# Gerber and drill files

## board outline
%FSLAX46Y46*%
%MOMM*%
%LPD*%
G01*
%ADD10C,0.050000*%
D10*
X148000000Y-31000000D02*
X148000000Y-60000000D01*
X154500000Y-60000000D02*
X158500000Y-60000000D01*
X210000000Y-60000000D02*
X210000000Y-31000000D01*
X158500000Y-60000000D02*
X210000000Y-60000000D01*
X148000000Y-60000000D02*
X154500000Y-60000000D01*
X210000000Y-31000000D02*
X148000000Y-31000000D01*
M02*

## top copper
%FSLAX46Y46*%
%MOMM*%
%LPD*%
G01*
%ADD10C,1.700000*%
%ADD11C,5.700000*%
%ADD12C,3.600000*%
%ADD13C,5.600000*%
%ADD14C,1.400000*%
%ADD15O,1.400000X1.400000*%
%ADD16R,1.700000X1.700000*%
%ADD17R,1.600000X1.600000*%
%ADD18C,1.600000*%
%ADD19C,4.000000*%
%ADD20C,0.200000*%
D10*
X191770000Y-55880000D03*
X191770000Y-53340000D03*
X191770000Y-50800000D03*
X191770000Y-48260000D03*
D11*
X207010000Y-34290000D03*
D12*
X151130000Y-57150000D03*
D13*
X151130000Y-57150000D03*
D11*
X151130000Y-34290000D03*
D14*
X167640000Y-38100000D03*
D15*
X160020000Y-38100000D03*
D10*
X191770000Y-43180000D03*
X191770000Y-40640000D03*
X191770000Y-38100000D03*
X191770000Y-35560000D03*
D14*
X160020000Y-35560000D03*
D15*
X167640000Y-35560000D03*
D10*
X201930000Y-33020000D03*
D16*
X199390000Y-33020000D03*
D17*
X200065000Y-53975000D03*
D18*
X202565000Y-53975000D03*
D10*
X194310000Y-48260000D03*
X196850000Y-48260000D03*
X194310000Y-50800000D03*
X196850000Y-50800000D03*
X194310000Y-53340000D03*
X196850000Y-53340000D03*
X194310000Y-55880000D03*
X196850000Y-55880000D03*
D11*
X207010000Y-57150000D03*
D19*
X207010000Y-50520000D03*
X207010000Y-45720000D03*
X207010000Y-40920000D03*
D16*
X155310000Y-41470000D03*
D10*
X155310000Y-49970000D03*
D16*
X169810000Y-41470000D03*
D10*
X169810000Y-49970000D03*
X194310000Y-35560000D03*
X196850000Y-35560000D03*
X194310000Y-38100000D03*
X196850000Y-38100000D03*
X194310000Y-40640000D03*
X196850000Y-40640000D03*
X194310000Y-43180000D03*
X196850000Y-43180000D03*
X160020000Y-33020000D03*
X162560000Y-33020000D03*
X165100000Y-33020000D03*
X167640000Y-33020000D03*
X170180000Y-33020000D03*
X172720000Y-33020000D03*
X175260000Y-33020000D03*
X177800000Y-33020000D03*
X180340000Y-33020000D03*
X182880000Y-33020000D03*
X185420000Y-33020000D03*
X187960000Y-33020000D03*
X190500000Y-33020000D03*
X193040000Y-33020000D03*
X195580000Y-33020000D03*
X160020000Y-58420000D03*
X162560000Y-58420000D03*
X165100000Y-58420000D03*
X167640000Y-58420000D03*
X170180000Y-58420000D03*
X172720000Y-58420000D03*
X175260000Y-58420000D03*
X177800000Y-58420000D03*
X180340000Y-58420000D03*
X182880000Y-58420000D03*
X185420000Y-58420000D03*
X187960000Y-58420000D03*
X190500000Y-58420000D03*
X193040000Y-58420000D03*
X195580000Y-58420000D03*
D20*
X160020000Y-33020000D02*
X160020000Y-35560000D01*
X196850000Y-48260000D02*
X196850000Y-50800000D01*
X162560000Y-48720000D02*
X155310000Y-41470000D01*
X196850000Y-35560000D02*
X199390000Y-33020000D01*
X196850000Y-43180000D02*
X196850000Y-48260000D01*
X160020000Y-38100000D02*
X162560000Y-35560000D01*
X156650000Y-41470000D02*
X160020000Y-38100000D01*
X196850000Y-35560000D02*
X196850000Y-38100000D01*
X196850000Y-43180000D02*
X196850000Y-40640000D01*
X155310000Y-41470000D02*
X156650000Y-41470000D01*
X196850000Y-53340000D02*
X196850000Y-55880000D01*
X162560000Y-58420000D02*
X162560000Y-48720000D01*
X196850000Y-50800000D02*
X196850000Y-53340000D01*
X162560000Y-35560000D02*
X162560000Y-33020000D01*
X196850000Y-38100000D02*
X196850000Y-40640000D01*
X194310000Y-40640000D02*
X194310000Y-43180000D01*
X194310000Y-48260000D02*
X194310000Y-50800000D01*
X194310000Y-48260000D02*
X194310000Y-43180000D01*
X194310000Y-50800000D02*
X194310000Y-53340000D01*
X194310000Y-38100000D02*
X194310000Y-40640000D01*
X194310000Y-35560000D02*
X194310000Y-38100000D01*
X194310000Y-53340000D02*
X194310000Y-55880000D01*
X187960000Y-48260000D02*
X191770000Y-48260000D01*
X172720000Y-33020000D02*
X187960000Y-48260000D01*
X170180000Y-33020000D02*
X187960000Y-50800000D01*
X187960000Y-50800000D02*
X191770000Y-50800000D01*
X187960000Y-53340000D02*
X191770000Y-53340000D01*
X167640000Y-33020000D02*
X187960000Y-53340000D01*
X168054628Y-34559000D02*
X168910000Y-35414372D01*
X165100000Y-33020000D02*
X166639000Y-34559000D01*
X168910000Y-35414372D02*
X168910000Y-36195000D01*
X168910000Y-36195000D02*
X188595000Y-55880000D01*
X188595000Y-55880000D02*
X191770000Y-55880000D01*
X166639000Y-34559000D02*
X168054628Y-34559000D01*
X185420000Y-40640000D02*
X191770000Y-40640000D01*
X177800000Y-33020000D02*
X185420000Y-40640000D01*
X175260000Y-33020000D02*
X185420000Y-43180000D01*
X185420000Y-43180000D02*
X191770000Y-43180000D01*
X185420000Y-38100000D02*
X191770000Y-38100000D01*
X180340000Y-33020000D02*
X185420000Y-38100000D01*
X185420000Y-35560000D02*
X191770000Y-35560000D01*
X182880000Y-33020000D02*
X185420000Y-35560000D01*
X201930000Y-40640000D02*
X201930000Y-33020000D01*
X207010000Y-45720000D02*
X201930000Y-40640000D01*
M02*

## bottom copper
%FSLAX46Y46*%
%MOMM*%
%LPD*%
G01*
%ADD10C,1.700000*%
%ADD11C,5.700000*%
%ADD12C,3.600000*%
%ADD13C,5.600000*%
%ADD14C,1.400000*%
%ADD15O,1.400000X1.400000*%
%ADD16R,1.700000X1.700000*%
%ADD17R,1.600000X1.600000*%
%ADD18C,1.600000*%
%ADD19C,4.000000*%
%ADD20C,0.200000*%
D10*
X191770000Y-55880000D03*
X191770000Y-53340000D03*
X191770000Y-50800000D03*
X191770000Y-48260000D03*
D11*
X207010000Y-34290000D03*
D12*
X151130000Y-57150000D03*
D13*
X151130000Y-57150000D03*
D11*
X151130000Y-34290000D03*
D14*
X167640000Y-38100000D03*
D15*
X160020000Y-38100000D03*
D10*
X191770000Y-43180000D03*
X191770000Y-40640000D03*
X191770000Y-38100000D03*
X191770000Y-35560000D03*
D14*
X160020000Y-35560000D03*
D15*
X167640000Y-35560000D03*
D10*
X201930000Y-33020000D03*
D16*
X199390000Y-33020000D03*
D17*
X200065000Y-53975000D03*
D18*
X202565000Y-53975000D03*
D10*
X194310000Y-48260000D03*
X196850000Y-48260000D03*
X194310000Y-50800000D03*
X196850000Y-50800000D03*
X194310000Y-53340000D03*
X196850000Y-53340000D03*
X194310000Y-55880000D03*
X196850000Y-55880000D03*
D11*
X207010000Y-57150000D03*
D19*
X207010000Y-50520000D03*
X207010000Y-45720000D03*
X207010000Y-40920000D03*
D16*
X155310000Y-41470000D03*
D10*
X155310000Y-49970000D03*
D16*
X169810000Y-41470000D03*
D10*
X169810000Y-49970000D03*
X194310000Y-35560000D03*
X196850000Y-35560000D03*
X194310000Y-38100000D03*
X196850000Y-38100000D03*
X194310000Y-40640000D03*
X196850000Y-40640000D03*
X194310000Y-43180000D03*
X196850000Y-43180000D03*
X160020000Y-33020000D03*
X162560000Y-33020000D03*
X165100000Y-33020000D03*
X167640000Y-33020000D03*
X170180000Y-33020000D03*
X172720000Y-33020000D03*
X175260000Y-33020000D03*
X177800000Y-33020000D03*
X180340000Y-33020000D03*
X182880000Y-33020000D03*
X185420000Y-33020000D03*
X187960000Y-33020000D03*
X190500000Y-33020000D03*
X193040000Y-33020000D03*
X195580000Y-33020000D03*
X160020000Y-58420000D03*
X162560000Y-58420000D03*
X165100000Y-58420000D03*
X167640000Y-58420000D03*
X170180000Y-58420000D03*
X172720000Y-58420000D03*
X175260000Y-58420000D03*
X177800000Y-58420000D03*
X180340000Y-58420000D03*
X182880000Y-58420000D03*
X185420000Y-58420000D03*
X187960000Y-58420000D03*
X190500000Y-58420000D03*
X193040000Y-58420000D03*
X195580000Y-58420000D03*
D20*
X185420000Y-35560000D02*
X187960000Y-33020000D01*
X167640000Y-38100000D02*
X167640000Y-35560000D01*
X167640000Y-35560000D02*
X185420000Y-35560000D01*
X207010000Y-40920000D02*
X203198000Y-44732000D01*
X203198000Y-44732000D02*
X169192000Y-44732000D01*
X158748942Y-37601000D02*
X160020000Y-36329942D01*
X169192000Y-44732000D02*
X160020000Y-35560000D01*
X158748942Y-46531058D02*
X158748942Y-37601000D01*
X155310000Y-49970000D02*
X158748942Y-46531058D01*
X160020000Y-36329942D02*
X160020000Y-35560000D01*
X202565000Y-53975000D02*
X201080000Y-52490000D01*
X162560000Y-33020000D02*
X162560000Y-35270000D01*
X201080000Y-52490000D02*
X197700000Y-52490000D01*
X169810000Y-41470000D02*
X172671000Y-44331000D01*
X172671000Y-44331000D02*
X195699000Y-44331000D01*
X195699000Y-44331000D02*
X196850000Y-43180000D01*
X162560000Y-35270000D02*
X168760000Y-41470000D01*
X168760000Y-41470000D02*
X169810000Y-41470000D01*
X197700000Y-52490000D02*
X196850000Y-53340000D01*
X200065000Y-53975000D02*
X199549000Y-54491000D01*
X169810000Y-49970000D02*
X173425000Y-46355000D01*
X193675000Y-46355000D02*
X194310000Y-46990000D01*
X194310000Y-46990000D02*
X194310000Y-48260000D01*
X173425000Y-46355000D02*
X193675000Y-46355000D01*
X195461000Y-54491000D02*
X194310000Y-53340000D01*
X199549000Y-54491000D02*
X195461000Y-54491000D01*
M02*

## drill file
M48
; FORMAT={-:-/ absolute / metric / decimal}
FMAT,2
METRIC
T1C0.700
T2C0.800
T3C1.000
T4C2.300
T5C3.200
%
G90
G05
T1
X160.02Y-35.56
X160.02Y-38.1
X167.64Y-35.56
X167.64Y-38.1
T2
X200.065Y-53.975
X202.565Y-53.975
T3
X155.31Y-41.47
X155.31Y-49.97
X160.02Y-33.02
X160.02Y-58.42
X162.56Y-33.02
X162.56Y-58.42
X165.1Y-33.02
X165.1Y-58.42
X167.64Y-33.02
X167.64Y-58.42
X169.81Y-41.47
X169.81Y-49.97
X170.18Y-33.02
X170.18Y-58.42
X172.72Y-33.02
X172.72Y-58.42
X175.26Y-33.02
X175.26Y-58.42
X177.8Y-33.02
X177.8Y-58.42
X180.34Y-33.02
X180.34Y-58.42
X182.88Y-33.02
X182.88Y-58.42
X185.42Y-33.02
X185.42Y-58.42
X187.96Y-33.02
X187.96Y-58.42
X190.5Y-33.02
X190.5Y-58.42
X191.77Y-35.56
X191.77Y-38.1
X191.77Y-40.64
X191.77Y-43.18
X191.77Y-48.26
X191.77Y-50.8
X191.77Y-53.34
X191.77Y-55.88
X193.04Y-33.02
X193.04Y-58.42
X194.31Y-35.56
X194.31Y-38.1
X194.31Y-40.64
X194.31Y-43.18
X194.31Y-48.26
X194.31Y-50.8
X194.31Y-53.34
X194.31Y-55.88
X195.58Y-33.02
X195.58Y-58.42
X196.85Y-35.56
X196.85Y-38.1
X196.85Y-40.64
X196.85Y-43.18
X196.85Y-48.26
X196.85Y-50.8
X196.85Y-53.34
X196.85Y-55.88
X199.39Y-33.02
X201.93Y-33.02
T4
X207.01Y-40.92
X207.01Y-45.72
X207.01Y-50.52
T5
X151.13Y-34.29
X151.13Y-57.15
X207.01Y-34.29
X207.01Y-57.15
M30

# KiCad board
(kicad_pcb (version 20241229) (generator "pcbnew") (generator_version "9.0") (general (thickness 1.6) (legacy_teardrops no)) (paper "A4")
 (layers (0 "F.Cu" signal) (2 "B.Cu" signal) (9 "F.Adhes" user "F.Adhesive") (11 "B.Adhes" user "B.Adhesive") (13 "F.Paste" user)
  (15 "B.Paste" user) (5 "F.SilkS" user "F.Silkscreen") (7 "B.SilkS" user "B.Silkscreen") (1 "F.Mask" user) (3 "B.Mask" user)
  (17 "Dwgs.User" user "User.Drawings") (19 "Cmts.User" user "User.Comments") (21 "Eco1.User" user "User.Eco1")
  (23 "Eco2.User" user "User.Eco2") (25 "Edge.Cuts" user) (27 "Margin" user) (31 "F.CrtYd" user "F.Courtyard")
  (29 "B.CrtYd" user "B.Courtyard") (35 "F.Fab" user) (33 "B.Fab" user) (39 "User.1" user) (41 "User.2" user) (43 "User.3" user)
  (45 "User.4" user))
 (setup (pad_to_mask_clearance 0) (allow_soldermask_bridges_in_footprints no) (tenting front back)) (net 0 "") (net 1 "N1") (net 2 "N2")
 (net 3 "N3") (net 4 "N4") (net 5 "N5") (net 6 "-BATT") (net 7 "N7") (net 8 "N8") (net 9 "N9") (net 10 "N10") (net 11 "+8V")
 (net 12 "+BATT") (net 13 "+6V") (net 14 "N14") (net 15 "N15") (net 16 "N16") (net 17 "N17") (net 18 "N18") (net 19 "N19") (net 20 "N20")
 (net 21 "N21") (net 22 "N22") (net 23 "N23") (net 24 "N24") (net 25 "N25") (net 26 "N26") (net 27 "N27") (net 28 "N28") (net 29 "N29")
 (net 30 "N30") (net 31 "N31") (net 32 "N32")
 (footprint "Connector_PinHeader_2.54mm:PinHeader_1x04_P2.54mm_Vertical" (layer "F.Cu") (at 191.77 55.88 180)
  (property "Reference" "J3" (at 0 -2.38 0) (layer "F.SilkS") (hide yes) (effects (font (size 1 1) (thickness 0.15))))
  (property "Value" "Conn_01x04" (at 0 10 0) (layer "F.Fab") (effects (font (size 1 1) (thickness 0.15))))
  (pad "1" thru_hole circle (at 0 0 180) (size 1.7 1.7) (drill 1) (layers "*.Cu" "*.Mask") (remove_unused_layers no) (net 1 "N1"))
  (pad "2" thru_hole circle (at 0 2.54 180) (size 1.7 1.7) (drill 1) (layers "*.Cu" "*.Mask") (remove_unused_layers no) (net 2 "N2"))
  (pad "3" thru_hole circle (at 0 5.08 180) (size 1.7 1.7) (drill 1) (layers "*.Cu" "*.Mask") (remove_unused_layers no) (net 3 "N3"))
  (pad "4" thru_hole circle (at 0 7.62 180) (size 1.7 1.7) (drill 1) (layers "*.Cu" "*.Mask") (remove_unused_layers no) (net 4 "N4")))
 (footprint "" (layer "F.Cu") (at 207.01 34.29)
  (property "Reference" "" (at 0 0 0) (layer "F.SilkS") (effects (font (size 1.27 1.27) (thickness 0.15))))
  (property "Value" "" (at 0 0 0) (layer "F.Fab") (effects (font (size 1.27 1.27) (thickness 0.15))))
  (pad "1" thru_hole circle (at 0 0) (size 5.7 5.7) (drill 3.2) (layers "*.Cu" "*.Mask") (remove_unused_layers no)))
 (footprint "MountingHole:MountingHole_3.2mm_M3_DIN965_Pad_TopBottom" (layer "F.Cu") (at 151.13 57.15)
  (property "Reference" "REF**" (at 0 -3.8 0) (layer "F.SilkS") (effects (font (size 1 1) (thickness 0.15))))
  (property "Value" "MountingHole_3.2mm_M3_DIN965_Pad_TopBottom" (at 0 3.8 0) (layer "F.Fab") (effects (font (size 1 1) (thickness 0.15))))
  (pad "1" thru_hole circle (at 0 0) (size 3.6 3.6) (drill 3.2) (layers "*.Cu" "*.Mask") (remove_unused_layers no))
  (pad "1" connect circle (at 0 0) (size 5.6 5.6) (layers "F.Cu" "F.Mask"))
  (pad "1" connect circle (at 0 0) (size 5.6 5.6) (layers "B.Cu" "B.Mask")))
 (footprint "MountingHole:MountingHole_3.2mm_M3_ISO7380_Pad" (layer "F.Cu") (at 151.13 34.29)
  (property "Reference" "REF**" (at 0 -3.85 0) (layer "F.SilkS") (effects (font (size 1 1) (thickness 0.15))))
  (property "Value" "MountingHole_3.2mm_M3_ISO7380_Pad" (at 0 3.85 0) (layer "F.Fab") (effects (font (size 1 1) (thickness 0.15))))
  (pad "1" thru_hole circle (at 0 0) (size 5.7 5.7) (drill 3.2) (layers "*.Cu" "*.Mask") (remove_unused_layers no)))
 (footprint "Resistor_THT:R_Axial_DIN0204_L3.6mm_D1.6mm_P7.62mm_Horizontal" (layer "F.Cu") (at 167.64 38.1 180)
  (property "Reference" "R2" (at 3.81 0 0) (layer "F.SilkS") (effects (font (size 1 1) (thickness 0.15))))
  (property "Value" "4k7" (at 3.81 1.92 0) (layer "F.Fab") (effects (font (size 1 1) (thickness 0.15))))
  (pad "1" thru_hole circle (at 0 0 180) (size 1.4 1.4) (drill 0.7) (layers "*.Cu" "*.Mask") (remove_unused_layers no) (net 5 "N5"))
  (pad "2" thru_hole oval (at 7.62 0 180) (size 1.4 1.4) (drill 0.7) (layers "*.Cu" "*.Mask") (remove_unused_layers no) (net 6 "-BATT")))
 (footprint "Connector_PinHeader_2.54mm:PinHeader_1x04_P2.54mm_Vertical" (layer "F.Cu") (at 191.77 43.18 180)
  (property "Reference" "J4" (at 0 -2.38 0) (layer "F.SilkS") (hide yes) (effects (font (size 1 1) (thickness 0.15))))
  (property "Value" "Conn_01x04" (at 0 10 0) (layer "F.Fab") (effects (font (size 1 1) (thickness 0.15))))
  (pad "1" thru_hole circle (at 0 0 180) (size 1.7 1.7) (drill 1) (layers "*.Cu" "*.Mask") (remove_unused_layers no) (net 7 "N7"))
  (pad "2" thru_hole circle (at 0 2.54 180) (size 1.7 1.7) (drill 1) (layers "*.Cu" "*.Mask") (remove_unused_layers no) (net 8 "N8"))
  (pad "3" thru_hole circle (at 0 5.08 180) (size 1.7 1.7) (drill 1) (layers "*.Cu" "*.Mask") (remove_unused_layers no) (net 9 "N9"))
  (pad "4" thru_hole circle (at 0 7.62 180) (size 1.7 1.7) (drill 1) (layers "*.Cu" "*.Mask") (remove_unused_layers no) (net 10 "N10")))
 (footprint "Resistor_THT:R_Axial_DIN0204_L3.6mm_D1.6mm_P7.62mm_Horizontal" (layer "F.Cu") (at 160.02 35.56)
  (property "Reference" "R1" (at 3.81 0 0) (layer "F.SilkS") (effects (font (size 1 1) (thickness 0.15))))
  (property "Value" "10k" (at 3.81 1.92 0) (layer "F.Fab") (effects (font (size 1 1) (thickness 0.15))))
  (pad "1" thru_hole circle (at 0 0) (size 1.4 1.4) (drill 0.7) (layers "*.Cu" "*.Mask") (remove_unused_layers no) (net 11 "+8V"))
  (pad "2" thru_hole oval (at 7.62 0) (size 1.4 1.4) (drill 0.7) (layers "*.Cu" "*.Mask") (remove_unused_layers no) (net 5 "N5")))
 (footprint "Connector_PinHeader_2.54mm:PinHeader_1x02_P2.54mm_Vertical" (layer "F.Cu") (at 201.93 33.02 -90)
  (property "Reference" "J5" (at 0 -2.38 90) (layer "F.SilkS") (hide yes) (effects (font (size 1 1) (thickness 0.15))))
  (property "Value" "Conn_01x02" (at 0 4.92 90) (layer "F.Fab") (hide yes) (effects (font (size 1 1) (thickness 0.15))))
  (pad "1" thru_hole circle (at 0 0 270) (size 1.7 1.7) (drill 1) (layers "*.Cu" "*.Mask") (remove_unused_layers no) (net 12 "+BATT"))
  (pad "2" thru_hole rect (at 0 2.54 270) (size 1.7 1.7) (drill 1) (layers "*.Cu" "*.Mask") (remove_unused_layers no) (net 6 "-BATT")))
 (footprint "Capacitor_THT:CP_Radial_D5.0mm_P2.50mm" (layer "F.Cu") (at 200.065 53.975)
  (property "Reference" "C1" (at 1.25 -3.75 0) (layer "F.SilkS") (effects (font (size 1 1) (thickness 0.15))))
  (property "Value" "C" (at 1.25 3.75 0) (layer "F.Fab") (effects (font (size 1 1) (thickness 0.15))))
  (pad "1" thru_hole rect (at 0 0) (size 1.6 1.6) (drill 0.8) (layers "*.Cu" "*.Mask") (remove_unused_layers no) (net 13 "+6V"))
  (pad "2" thru_hole circle (at 2.5 0) (size 1.6 1.6) (drill 0.8) (layers "*.Cu" "*.Mask") (remove_unused_layers no) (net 6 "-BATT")))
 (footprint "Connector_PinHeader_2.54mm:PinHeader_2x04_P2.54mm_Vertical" (layer "F.Cu") (at 194.31 48.26)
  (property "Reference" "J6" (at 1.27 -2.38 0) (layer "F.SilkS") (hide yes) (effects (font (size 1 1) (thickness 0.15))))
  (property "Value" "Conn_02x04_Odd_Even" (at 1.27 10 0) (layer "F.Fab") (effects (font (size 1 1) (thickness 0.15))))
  (pad "1" thru_hole circle (at 0 0) (size 1.7 1.7) (drill 1) (layers "*.Cu" "*.Mask") (remove_unused_layers no) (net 13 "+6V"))
  (pad "2" thru_hole circle (at 2.54 0) (size 1.7 1.7) (drill 1) (layers "*.Cu" "*.Mask") (remove_unused_layers no) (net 6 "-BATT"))
  (pad "3" thru_hole circle (at 0 2.54) (size 1.7 1.7) (drill 1) (layers "*.Cu" "*.Mask") (remove_unused_layers no) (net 13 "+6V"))
  (pad "4" thru_hole circle (at 2.54 2.54) (size 1.7 1.7) (drill 1) (layers "*.Cu" "*.Mask") (remove_unused_layers no) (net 6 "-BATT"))
  (pad "5" thru_hole circle (at 0 5.08) (size 1.7 1.7) (drill 1) (layers "*.Cu" "*.Mask") (remove_unused_layers no) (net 13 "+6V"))
  (pad "6" thru_hole circle (at 2.54 5.08) (size 1.7 1.7) (drill 1) (layers "*.Cu" "*.Mask") (remove_unused_layers no) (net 6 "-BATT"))
  (pad "7" thru_hole circle (at 0 7.62) (size 1.7 1.7) (drill 1) (layers "*.Cu" "*.Mask") (remove_unused_layers no) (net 13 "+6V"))
  (pad "8" thru_hole circle (at 2.54 7.62) (size 1.7 1.7) (drill 1) (layers "*.Cu" "*.Mask") (remove_unused_layers no) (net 6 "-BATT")))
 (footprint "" (layer "F.Cu") (at 207.01 57.15)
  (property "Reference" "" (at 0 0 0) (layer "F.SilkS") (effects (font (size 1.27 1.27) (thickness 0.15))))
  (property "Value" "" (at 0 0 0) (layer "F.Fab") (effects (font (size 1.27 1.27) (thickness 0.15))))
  (pad "1" thru_hole circle (at 0 0) (size 5.7 5.7) (drill 3.2) (layers "*.Cu" "*.Mask") (remove_unused_layers no)))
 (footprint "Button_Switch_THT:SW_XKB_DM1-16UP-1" (layer "F.Cu") (at 207.01 50.52 90)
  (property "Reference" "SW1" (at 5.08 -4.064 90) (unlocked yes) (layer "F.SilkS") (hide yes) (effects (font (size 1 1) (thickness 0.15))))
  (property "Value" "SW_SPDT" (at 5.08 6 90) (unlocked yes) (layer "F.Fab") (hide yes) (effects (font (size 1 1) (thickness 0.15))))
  (pad "1" thru_hole circle (at 0 0 90) (size 4 4) (drill 2.3) (layers "*.Cu" "*.Mask") (remove_unused_layers no) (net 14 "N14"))
  (pad "2" thru_hole circle (at 4.8 0 90) (size 4 4) (drill 2.3) (layers "*.Cu" "*.Mask") (remove_unused_layers no) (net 12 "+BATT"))
  (pad "3" thru_hole circle (at 9.6 0 90) (size 4 4) (drill 2.3) (layers "*.Cu" "*.Mask") (remove_unused_layers no) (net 11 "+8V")))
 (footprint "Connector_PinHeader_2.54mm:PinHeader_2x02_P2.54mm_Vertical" (layer "F.Cu") (at 169.81 41.47 -90)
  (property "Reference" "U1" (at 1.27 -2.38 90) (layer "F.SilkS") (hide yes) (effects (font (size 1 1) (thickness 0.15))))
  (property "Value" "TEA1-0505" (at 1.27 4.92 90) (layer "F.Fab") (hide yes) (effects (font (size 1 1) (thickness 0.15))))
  (pad "1" thru_hole rect (at 0 14.5 270) (size 1.7 1.7) (drill 1) (layers "*.Cu" "*.Mask") (remove_unused_layers no) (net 6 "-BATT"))
  (pad "2" thru_hole circle (at 8.5 14.5 270) (size 1.7 1.7) (drill 1) (layers "*.Cu" "*.Mask") (remove_unused_layers no) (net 11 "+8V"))
  (pad "3" thru_hole rect (at 0 0 270) (size 1.7 1.7) (drill 1) (layers "*.Cu" "*.Mask") (remove_unused_layers no) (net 6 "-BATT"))
  (pad "4" thru_hole circle (at 8.5 0 270) (size 1.7 1.7) (drill 1) (layers "*.Cu" "*.Mask") (remove_unused_layers no) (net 13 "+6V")))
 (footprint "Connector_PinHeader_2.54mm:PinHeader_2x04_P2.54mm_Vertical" (layer "F.Cu") (at 194.31 35.56)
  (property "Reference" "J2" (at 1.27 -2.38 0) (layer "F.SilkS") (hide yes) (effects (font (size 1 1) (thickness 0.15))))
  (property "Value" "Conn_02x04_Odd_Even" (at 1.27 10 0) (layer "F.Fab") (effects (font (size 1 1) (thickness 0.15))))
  (pad "1" thru_hole circle (at 0 0) (size 1.7 1.7) (drill 1) (layers "*.Cu" "*.Mask") (remove_unused_layers no) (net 13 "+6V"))
  (pad "2" thru_hole circle (at 2.54 0) (size 1.7 1.7) (drill 1) (layers "*.Cu" "*.Mask") (remove_unused_layers no) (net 6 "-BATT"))
  (pad "3" thru_hole circle (at 0 2.54) (size 1.7 1.7) (drill 1) (layers "*.Cu" "*.Mask") (remove_unused_layers no) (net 13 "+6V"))
  (pad "4" thru_hole circle (at 2.54 2.54) (size 1.7 1.7) (drill 1) (layers "*.Cu" "*.Mask") (remove_unused_layers no) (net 6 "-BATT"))
  (pad "5" thru_hole circle (at 0 5.08) (size 1.7 1.7) (drill 1) (layers "*.Cu" "*.Mask") (remove_unused_layers no) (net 13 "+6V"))
  (pad "6" thru_hole circle (at 2.54 5.08) (size 1.7 1.7) (drill 1) (layers "*.Cu" "*.Mask") (remove_unused_layers no) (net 6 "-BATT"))
  (pad "7" thru_hole circle (at 0 7.62) (size 1.7 1.7) (drill 1) (layers "*.Cu" "*.Mask") (remove_unused_layers no) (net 13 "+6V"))
  (pad "8" thru_hole circle (at 2.54 7.62) (size 1.7 1.7) (drill 1) (layers "*.Cu" "*.Mask") (remove_unused_layers no) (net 6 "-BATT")))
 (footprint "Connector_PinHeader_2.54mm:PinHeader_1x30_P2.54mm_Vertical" (layer "B.Cu") (at 160.02 33.02 -90)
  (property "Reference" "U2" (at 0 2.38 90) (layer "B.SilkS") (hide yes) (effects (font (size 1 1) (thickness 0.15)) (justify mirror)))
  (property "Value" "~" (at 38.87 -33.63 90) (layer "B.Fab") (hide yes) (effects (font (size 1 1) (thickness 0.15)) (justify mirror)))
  (pad "1" thru_hole circle (at 0 0 270) (size 1.7 1.7) (drill 1) (layers "*.Cu" "*.Mask") (remove_unused_layers no) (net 11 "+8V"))
  (pad "2" thru_hole circle (at 0 -2.54 270) (size 1.7 1.7) (drill 1) (layers "*.Cu" "*.Mask") (remove_unused_layers no) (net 6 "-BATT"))
  (pad "3" thru_hole circle (at 0 -5.08 270) (size 1.7 1.7) (drill 1) (layers "*.Cu" "*.Mask") (remove_unused_layers no) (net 1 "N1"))
  (pad "4" thru_hole circle (at 0 -7.62 270) (size 1.7 1.7) (drill 1) (layers "*.Cu" "*.Mask") (remove_unused_layers no) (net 2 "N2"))
  (pad "5" thru_hole circle (at 0 -10.16 270) (size 1.7 1.7) (drill 1) (layers "*.Cu" "*.Mask") (remove_unused_layers no) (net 3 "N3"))
  (pad "6" thru_hole circle (at 0 -12.7 270) (size 1.7 1.7) (drill 1) (layers "*.Cu" "*.Mask") (remove_unused_layers no) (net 4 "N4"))
  (pad "7" thru_hole circle (at 0 -15.24 270) (size 1.7 1.7) (drill 1) (layers "*.Cu" "*.Mask") (remove_unused_layers no) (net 7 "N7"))
  (pad "8" thru_hole circle (at 0 -17.78 270) (size 1.7 1.7) (drill 1) (layers "*.Cu" "*.Mask") (remove_unused_layers no) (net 8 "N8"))
  (pad "9" thru_hole circle (at 0 -20.32 270) (size 1.7 1.7) (drill 1) (layers "*.Cu" "*.Mask") (remove_unused_layers no) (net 9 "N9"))
  (pad "10" thru_hole circle (at 0 -22.86 270) (size 1.7 1.7) (drill 1) (layers "*.Cu" "*.Mask") (remove_unused_layers no) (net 10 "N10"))
  (pad "11" thru_hole circle (at 0 -25.4 270) (size 1.7 1.7) (drill 1) (layers "*.Cu" "*.Mask") (remove_unused_layers no) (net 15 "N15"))
  (pad "12" thru_hole circle (at 0 -27.94 270) (size 1.7 1.7) (drill 1) (layers "*.Cu" "*.Mask") (remove_unused_layers no) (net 5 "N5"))
  (pad "13" thru_hole circle (at 0 -30.48 270) (size 1.7 1.7) (drill 1) (layers "*.Cu" "*.Mask") (remove_unused_layers no) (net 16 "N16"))
  (pad "14" thru_hole circle (at 0 -33.02 270) (size 1.7 1.7) (drill 1) (layers "*.Cu" "*.Mask") (remove_unused_layers no) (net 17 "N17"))
  (pad "15" thru_hole circle (at 0 -35.56 270) (size 1.7 1.7) (drill 1) (layers "*.Cu" "*.Mask") (remove_unused_layers no) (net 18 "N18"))
  (pad "16" thru_hole circle (at 25.4 0 270) (size 1.7 1.7) (drill 1) (layers "*.Cu" "*.Mask") (remove_unused_layers no) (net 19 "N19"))
  (pad "17" thru_hole circle (at 25.4 -2.54 270) (size 1.7 1.7) (drill 1) (layers "*.Cu" "*.Mask") (remove_unused_layers no) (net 6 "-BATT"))
  (pad "18" thru_hole circle (at 25.4 -5.08 270) (size 1.7 1.7) (drill 1) (layers "*.Cu" "*.Mask") (remove_unused_layers no) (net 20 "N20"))
  (pad "19" thru_hole circle (at 25.4 -7.62 270) (size 1.7 1.7) (drill 1) (layers "*.Cu" "*.Mask") (remove_unused_layers no) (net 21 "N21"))
  (pad "20" thru_hole circle (at 25.4 -10.16 270) (size 1.7 1.7) (drill 1) (layers "*.Cu" "*.Mask") (remove_unused_layers no) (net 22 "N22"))
  (pad "21" thru_hole circle (at 25.4 -12.7 270) (size 1.7 1.7) (drill 1) (layers "*.Cu" "*.Mask") (remove_unused_layers no) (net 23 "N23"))
  (pad "22" thru_hole circle (at 25.4 -15.24 270) (size 1.7 1.7) (drill 1) (layers "*.Cu" "*.Mask") (remove_unused_layers no) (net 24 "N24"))
  (pad "23" thru_hole circle (at 25.4 -17.78 270) (size 1.7 1.7) (drill 1) (layers "*.Cu" "*.Mask") (remove_unused_layers no) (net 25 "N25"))
  (pad "24" thru_hole circle (at 25.4 -20.32 270) (size 1.7 1.7) (drill 1) (layers "*.Cu" "*.Mask") (remove_unused_layers no) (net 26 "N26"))
  (pad "25" thru_hole circle (at 25.4 -22.86 270) (size 1.7 1.7) (drill 1) (layers "*.Cu" "*.Mask") (remove_unused_layers no) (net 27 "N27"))
  (pad "26" thru_hole circle (at 25.4 -25.4 270) (size 1.7 1.7) (drill 1) (layers "*.Cu" "*.Mask") (remove_unused_layers no) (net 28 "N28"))
  (pad "27" thru_hole circle (at 25.4 -27.94 270) (size 1.7 1.7) (drill 1) (layers "*.Cu" "*.Mask") (remove_unused_layers no) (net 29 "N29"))
  (pad "28" thru_hole circle (at 25.4 -30.48 270) (size 1.7 1.7) (drill 1) (layers "*.Cu" "*.Mask") (remove_unused_layers no) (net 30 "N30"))
  (pad "29" thru_hole circle (at 25.4 -33.02 270) (size 1.7 1.7) (drill 1) (layers "*.Cu" "*.Mask") (remove_unused_layers no) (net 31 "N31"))
  (pad "30" thru_hole circle (at 25.4 -35.56 270) (size 1.7 1.7) (drill 1) (layers "*.Cu" "*.Mask") (remove_unused_layers no) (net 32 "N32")))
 (gr_line (start 148 31) (end 148 60) (stroke (width 0.05) (type default)) (layer "Edge.Cuts"))
 (gr_line (start 154.5 60) (end 158.5 60) (stroke (width 0.05) (type default)) (layer "Edge.Cuts"))
 (gr_line (start 210 60) (end 210 31) (stroke (width 0.05) (type default)) (layer "Edge.Cuts"))
 (gr_line (start 158.5 60) (end 210 60) (stroke (width 0.05) (type default)) (layer "Edge.Cuts"))
 (gr_line (start 148 60) (end 154.5 60) (stroke (width 0.05) (type default)) (layer "Edge.Cuts"))
 (gr_line (start 210 31) (end 148 31) (stroke (width 0.05) (type default)) (layer "Edge.Cuts"))
 (segment (start 185.42 35.56) (end 187.96 33.02) (width 0.2) (layer "B.Cu") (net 5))
 (segment (start 167.64 38.1) (end 167.64 35.56) (width 0.2) (layer "B.Cu") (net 5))
 (segment (start 167.64 35.56) (end 185.42 35.56) (width 0.2) (layer "B.Cu") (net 5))
 (segment (start 160.02 33.02) (end 160.02 35.56) (width 0.2) (layer "F.Cu") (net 11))
 (segment (start 207.01 40.92) (end 203.198 44.732) (width 0.2) (layer "B.Cu") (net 11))
 (segment (start 203.198 44.732) (end 169.192 44.732) (width 0.2) (layer "B.Cu") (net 11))
 (segment (start 158.748942 37.601) (end 160.02 36.329942) (width 0.2) (layer "B.Cu") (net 11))
 (segment (start 169.192 44.732) (end 160.02 35.56) (width 0.2) (layer "B.Cu") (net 11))
 (segment (start 158.748942 46.531058) (end 158.748942 37.601) (width 0.2) (layer "B.Cu") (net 11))
 (segment (start 155.31 49.97) (end 158.748942 46.531058) (width 0.2) (layer "B.Cu") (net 11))
 (segment (start 160.02 36.329942) (end 160.02 35.56) (width 0.2) (layer "B.Cu") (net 11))
 (segment (start 196.85 48.26) (end 196.85 50.8) (width 0.2) (layer "F.Cu") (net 6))
 (segment (start 162.56 48.72) (end 155.31 41.47) (width 0.2) (layer "F.Cu") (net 6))
 (segment (start 196.85 35.56) (end 199.39 33.02) (width 0.2) (layer "F.Cu") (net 6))
 (segment (start 196.85 43.18) (end 196.85 48.26) (width 0.2) (layer "F.Cu") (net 6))
 (segment (start 160.02 38.1) (end 162.56 35.56) (width 0.2) (layer "F.Cu") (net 6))
 (segment (start 156.65 41.47) (end 160.02 38.1) (width 0.2) (layer "F.Cu") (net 6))
 (segment (start 196.85 35.56) (end 196.85 38.1) (width 0.2) (layer "F.Cu") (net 6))
 (segment (start 196.85 43.18) (end 196.85 40.64) (width 0.2) (layer "F.Cu") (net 6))
 (segment (start 155.31 41.47) (end 156.65 41.47) (width 0.2) (layer "F.Cu") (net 6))
 (segment (start 196.85 53.34) (end 196.85 55.88) (width 0.2) (layer "F.Cu") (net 6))
 (segment (start 162.56 58.42) (end 162.56 48.72) (width 0.2) (layer "F.Cu") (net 6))
 (segment (start 196.85 50.8) (end 196.85 53.34) (width 0.2) (layer "F.Cu") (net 6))
 (segment (start 162.56 35.56) (end 162.56 33.02) (width 0.2) (layer "F.Cu") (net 6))
 (segment (start 196.85 38.1) (end 196.85 40.64) (width 0.2) (layer "F.Cu") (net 6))
 (segment (start 202.565 53.975) (end 201.08 52.49) (width 0.2) (layer "B.Cu") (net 6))
 (segment (start 162.56 33.02) (end 162.56 35.27) (width 0.2) (layer "B.Cu") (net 6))
 (segment (start 201.08 52.49) (end 197.7 52.49) (width 0.2) (layer "B.Cu") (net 6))
 (segment (start 169.81 41.47) (end 172.671 44.331) (width 0.2) (layer "B.Cu") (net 6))
 (segment (start 172.671 44.331) (end 195.699 44.331) (width 0.2) (layer "B.Cu") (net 6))
 (segment (start 195.699 44.331) (end 196.85 43.18) (width 0.2) (layer "B.Cu") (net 6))
 (segment (start 162.56 35.27) (end 168.76 41.47) (width 0.2) (layer "B.Cu") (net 6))
 (segment (start 168.76 41.47) (end 169.81 41.47) (width 0.2) (layer "B.Cu") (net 6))
 (segment (start 197.7 52.49) (end 196.85 53.34) (width 0.2) (layer "B.Cu") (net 6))
 (segment (start 194.31 40.64) (end 194.31 43.18) (width 0.2) (layer "F.Cu") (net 13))
 (segment (start 194.31 48.26) (end 194.31 50.8) (width 0.2) (layer "F.Cu") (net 13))
 (segment (start 194.31 48.26) (end 194.31 43.18) (width 0.2) (layer "F.Cu") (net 13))
 (segment (start 194.31 50.8) (end 194.31 53.34) (width 0.2) (layer "F.Cu") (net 13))
 (segment (start 194.31 38.1) (end 194.31 40.64) (width 0.2) (layer "F.Cu") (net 13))
 (segment (start 194.31 35.56) (end 194.31 38.1) (width 0.2) (layer "F.Cu") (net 13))
 (segment (start 194.31 53.34) (end 194.31 55.88) (width 0.2) (layer "F.Cu") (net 13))
 (segment (start 200.065 53.975) (end 199.549 54.491) (width 0.2) (layer "B.Cu") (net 13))
 (segment (start 169.81 49.97) (end 173.425 46.355) (width 0.2) (layer "B.Cu") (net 13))
 (segment (start 193.675 46.355) (end 194.31 46.99) (width 0.2) (layer "B.Cu") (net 13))
 (segment (start 194.31 46.99) (end 194.31 48.26) (width 0.2) (layer "B.Cu") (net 13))
 (segment (start 173.425 46.355) (end 193.675 46.355) (width 0.2) (layer "B.Cu") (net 13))
 (segment (start 195.461 54.491) (end 194.31 53.34) (width 0.2) (layer "B.Cu") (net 13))
 (segment (start 199.549 54.491) (end 195.461 54.491) (width 0.2) (layer "B.Cu") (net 13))
 (segment (start 187.96 48.26) (end 191.77 48.26) (width 0.2) (layer "F.Cu") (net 4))
 (segment (start 172.72 33.02) (end 187.96 48.26) (width 0.2) (layer "F.Cu") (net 4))
 (segment (start 170.18 33.02) (end 187.96 50.8) (width 0.2) (layer "F.Cu") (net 3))
 (segment (start 187.96 50.8) (end 191.77 50.8) (width 0.2) (layer "F.Cu") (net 3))
 (segment (start 187.96 53.34) (end 191.77 53.34) (width 0.2) (layer "F.Cu") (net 2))
 (segment (start 167.64 33.02) (end 187.96 53.34) (width 0.2) (layer "F.Cu") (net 2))
 (segment (start 168.054628 34.559) (end 168.91 35.414372) (width 0.2) (layer "F.Cu") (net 1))
 (segment (start 165.1 33.02) (end 166.639 34.559) (width 0.2) (layer "F.Cu") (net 1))
 (segment (start 168.91 35.414372) (end 168.91 36.195) (width 0.2) (layer "F.Cu") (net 1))
 (segment (start 168.91 36.195) (end 188.595 55.88) (width 0.2) (layer "F.Cu") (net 1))
 (segment (start 188.595 55.88) (end 191.77 55.88) (width 0.2) (layer "F.Cu") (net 1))
 (segment (start 166.639 34.559) (end 168.054628 34.559) (width 0.2) (layer "F.Cu") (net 1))
 (segment (start 185.42 40.64) (end 191.77 40.64) (width 0.2) (layer "F.Cu") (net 8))
 (segment (start 177.8 33.02) (end 185.42 40.64) (width 0.2) (layer "F.Cu") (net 8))
 (segment (start 175.26 33.02) (end 185.42 43.18) (width 0.2) (layer "F.Cu") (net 7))
 (segment (start 185.42 43.18) (end 191.77 43.18) (width 0.2) (layer "F.Cu") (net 7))
 (segment (start 185.42 38.1) (end 191.77 38.1) (width 0.2) (layer "F.Cu") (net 9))
 (segment (start 180.34 33.02) (end 185.42 38.1) (width 0.2) (layer "F.Cu") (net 9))
 (segment (start 185.42 35.56) (end 191.77 35.56) (width 0.2) (layer "F.Cu") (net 10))
 (segment (start 182.88 33.02) (end 185.42 35.56) (width 0.2) (layer "F.Cu") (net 10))
 (segment (start 201.93 40.64) (end 201.93 33.02) (width 0.2) (layer "F.Cu") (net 12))
 (segment (start 207.01 45.72) (end 201.93 40.64) (width 0.2) (layer "F.Cu") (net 12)))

